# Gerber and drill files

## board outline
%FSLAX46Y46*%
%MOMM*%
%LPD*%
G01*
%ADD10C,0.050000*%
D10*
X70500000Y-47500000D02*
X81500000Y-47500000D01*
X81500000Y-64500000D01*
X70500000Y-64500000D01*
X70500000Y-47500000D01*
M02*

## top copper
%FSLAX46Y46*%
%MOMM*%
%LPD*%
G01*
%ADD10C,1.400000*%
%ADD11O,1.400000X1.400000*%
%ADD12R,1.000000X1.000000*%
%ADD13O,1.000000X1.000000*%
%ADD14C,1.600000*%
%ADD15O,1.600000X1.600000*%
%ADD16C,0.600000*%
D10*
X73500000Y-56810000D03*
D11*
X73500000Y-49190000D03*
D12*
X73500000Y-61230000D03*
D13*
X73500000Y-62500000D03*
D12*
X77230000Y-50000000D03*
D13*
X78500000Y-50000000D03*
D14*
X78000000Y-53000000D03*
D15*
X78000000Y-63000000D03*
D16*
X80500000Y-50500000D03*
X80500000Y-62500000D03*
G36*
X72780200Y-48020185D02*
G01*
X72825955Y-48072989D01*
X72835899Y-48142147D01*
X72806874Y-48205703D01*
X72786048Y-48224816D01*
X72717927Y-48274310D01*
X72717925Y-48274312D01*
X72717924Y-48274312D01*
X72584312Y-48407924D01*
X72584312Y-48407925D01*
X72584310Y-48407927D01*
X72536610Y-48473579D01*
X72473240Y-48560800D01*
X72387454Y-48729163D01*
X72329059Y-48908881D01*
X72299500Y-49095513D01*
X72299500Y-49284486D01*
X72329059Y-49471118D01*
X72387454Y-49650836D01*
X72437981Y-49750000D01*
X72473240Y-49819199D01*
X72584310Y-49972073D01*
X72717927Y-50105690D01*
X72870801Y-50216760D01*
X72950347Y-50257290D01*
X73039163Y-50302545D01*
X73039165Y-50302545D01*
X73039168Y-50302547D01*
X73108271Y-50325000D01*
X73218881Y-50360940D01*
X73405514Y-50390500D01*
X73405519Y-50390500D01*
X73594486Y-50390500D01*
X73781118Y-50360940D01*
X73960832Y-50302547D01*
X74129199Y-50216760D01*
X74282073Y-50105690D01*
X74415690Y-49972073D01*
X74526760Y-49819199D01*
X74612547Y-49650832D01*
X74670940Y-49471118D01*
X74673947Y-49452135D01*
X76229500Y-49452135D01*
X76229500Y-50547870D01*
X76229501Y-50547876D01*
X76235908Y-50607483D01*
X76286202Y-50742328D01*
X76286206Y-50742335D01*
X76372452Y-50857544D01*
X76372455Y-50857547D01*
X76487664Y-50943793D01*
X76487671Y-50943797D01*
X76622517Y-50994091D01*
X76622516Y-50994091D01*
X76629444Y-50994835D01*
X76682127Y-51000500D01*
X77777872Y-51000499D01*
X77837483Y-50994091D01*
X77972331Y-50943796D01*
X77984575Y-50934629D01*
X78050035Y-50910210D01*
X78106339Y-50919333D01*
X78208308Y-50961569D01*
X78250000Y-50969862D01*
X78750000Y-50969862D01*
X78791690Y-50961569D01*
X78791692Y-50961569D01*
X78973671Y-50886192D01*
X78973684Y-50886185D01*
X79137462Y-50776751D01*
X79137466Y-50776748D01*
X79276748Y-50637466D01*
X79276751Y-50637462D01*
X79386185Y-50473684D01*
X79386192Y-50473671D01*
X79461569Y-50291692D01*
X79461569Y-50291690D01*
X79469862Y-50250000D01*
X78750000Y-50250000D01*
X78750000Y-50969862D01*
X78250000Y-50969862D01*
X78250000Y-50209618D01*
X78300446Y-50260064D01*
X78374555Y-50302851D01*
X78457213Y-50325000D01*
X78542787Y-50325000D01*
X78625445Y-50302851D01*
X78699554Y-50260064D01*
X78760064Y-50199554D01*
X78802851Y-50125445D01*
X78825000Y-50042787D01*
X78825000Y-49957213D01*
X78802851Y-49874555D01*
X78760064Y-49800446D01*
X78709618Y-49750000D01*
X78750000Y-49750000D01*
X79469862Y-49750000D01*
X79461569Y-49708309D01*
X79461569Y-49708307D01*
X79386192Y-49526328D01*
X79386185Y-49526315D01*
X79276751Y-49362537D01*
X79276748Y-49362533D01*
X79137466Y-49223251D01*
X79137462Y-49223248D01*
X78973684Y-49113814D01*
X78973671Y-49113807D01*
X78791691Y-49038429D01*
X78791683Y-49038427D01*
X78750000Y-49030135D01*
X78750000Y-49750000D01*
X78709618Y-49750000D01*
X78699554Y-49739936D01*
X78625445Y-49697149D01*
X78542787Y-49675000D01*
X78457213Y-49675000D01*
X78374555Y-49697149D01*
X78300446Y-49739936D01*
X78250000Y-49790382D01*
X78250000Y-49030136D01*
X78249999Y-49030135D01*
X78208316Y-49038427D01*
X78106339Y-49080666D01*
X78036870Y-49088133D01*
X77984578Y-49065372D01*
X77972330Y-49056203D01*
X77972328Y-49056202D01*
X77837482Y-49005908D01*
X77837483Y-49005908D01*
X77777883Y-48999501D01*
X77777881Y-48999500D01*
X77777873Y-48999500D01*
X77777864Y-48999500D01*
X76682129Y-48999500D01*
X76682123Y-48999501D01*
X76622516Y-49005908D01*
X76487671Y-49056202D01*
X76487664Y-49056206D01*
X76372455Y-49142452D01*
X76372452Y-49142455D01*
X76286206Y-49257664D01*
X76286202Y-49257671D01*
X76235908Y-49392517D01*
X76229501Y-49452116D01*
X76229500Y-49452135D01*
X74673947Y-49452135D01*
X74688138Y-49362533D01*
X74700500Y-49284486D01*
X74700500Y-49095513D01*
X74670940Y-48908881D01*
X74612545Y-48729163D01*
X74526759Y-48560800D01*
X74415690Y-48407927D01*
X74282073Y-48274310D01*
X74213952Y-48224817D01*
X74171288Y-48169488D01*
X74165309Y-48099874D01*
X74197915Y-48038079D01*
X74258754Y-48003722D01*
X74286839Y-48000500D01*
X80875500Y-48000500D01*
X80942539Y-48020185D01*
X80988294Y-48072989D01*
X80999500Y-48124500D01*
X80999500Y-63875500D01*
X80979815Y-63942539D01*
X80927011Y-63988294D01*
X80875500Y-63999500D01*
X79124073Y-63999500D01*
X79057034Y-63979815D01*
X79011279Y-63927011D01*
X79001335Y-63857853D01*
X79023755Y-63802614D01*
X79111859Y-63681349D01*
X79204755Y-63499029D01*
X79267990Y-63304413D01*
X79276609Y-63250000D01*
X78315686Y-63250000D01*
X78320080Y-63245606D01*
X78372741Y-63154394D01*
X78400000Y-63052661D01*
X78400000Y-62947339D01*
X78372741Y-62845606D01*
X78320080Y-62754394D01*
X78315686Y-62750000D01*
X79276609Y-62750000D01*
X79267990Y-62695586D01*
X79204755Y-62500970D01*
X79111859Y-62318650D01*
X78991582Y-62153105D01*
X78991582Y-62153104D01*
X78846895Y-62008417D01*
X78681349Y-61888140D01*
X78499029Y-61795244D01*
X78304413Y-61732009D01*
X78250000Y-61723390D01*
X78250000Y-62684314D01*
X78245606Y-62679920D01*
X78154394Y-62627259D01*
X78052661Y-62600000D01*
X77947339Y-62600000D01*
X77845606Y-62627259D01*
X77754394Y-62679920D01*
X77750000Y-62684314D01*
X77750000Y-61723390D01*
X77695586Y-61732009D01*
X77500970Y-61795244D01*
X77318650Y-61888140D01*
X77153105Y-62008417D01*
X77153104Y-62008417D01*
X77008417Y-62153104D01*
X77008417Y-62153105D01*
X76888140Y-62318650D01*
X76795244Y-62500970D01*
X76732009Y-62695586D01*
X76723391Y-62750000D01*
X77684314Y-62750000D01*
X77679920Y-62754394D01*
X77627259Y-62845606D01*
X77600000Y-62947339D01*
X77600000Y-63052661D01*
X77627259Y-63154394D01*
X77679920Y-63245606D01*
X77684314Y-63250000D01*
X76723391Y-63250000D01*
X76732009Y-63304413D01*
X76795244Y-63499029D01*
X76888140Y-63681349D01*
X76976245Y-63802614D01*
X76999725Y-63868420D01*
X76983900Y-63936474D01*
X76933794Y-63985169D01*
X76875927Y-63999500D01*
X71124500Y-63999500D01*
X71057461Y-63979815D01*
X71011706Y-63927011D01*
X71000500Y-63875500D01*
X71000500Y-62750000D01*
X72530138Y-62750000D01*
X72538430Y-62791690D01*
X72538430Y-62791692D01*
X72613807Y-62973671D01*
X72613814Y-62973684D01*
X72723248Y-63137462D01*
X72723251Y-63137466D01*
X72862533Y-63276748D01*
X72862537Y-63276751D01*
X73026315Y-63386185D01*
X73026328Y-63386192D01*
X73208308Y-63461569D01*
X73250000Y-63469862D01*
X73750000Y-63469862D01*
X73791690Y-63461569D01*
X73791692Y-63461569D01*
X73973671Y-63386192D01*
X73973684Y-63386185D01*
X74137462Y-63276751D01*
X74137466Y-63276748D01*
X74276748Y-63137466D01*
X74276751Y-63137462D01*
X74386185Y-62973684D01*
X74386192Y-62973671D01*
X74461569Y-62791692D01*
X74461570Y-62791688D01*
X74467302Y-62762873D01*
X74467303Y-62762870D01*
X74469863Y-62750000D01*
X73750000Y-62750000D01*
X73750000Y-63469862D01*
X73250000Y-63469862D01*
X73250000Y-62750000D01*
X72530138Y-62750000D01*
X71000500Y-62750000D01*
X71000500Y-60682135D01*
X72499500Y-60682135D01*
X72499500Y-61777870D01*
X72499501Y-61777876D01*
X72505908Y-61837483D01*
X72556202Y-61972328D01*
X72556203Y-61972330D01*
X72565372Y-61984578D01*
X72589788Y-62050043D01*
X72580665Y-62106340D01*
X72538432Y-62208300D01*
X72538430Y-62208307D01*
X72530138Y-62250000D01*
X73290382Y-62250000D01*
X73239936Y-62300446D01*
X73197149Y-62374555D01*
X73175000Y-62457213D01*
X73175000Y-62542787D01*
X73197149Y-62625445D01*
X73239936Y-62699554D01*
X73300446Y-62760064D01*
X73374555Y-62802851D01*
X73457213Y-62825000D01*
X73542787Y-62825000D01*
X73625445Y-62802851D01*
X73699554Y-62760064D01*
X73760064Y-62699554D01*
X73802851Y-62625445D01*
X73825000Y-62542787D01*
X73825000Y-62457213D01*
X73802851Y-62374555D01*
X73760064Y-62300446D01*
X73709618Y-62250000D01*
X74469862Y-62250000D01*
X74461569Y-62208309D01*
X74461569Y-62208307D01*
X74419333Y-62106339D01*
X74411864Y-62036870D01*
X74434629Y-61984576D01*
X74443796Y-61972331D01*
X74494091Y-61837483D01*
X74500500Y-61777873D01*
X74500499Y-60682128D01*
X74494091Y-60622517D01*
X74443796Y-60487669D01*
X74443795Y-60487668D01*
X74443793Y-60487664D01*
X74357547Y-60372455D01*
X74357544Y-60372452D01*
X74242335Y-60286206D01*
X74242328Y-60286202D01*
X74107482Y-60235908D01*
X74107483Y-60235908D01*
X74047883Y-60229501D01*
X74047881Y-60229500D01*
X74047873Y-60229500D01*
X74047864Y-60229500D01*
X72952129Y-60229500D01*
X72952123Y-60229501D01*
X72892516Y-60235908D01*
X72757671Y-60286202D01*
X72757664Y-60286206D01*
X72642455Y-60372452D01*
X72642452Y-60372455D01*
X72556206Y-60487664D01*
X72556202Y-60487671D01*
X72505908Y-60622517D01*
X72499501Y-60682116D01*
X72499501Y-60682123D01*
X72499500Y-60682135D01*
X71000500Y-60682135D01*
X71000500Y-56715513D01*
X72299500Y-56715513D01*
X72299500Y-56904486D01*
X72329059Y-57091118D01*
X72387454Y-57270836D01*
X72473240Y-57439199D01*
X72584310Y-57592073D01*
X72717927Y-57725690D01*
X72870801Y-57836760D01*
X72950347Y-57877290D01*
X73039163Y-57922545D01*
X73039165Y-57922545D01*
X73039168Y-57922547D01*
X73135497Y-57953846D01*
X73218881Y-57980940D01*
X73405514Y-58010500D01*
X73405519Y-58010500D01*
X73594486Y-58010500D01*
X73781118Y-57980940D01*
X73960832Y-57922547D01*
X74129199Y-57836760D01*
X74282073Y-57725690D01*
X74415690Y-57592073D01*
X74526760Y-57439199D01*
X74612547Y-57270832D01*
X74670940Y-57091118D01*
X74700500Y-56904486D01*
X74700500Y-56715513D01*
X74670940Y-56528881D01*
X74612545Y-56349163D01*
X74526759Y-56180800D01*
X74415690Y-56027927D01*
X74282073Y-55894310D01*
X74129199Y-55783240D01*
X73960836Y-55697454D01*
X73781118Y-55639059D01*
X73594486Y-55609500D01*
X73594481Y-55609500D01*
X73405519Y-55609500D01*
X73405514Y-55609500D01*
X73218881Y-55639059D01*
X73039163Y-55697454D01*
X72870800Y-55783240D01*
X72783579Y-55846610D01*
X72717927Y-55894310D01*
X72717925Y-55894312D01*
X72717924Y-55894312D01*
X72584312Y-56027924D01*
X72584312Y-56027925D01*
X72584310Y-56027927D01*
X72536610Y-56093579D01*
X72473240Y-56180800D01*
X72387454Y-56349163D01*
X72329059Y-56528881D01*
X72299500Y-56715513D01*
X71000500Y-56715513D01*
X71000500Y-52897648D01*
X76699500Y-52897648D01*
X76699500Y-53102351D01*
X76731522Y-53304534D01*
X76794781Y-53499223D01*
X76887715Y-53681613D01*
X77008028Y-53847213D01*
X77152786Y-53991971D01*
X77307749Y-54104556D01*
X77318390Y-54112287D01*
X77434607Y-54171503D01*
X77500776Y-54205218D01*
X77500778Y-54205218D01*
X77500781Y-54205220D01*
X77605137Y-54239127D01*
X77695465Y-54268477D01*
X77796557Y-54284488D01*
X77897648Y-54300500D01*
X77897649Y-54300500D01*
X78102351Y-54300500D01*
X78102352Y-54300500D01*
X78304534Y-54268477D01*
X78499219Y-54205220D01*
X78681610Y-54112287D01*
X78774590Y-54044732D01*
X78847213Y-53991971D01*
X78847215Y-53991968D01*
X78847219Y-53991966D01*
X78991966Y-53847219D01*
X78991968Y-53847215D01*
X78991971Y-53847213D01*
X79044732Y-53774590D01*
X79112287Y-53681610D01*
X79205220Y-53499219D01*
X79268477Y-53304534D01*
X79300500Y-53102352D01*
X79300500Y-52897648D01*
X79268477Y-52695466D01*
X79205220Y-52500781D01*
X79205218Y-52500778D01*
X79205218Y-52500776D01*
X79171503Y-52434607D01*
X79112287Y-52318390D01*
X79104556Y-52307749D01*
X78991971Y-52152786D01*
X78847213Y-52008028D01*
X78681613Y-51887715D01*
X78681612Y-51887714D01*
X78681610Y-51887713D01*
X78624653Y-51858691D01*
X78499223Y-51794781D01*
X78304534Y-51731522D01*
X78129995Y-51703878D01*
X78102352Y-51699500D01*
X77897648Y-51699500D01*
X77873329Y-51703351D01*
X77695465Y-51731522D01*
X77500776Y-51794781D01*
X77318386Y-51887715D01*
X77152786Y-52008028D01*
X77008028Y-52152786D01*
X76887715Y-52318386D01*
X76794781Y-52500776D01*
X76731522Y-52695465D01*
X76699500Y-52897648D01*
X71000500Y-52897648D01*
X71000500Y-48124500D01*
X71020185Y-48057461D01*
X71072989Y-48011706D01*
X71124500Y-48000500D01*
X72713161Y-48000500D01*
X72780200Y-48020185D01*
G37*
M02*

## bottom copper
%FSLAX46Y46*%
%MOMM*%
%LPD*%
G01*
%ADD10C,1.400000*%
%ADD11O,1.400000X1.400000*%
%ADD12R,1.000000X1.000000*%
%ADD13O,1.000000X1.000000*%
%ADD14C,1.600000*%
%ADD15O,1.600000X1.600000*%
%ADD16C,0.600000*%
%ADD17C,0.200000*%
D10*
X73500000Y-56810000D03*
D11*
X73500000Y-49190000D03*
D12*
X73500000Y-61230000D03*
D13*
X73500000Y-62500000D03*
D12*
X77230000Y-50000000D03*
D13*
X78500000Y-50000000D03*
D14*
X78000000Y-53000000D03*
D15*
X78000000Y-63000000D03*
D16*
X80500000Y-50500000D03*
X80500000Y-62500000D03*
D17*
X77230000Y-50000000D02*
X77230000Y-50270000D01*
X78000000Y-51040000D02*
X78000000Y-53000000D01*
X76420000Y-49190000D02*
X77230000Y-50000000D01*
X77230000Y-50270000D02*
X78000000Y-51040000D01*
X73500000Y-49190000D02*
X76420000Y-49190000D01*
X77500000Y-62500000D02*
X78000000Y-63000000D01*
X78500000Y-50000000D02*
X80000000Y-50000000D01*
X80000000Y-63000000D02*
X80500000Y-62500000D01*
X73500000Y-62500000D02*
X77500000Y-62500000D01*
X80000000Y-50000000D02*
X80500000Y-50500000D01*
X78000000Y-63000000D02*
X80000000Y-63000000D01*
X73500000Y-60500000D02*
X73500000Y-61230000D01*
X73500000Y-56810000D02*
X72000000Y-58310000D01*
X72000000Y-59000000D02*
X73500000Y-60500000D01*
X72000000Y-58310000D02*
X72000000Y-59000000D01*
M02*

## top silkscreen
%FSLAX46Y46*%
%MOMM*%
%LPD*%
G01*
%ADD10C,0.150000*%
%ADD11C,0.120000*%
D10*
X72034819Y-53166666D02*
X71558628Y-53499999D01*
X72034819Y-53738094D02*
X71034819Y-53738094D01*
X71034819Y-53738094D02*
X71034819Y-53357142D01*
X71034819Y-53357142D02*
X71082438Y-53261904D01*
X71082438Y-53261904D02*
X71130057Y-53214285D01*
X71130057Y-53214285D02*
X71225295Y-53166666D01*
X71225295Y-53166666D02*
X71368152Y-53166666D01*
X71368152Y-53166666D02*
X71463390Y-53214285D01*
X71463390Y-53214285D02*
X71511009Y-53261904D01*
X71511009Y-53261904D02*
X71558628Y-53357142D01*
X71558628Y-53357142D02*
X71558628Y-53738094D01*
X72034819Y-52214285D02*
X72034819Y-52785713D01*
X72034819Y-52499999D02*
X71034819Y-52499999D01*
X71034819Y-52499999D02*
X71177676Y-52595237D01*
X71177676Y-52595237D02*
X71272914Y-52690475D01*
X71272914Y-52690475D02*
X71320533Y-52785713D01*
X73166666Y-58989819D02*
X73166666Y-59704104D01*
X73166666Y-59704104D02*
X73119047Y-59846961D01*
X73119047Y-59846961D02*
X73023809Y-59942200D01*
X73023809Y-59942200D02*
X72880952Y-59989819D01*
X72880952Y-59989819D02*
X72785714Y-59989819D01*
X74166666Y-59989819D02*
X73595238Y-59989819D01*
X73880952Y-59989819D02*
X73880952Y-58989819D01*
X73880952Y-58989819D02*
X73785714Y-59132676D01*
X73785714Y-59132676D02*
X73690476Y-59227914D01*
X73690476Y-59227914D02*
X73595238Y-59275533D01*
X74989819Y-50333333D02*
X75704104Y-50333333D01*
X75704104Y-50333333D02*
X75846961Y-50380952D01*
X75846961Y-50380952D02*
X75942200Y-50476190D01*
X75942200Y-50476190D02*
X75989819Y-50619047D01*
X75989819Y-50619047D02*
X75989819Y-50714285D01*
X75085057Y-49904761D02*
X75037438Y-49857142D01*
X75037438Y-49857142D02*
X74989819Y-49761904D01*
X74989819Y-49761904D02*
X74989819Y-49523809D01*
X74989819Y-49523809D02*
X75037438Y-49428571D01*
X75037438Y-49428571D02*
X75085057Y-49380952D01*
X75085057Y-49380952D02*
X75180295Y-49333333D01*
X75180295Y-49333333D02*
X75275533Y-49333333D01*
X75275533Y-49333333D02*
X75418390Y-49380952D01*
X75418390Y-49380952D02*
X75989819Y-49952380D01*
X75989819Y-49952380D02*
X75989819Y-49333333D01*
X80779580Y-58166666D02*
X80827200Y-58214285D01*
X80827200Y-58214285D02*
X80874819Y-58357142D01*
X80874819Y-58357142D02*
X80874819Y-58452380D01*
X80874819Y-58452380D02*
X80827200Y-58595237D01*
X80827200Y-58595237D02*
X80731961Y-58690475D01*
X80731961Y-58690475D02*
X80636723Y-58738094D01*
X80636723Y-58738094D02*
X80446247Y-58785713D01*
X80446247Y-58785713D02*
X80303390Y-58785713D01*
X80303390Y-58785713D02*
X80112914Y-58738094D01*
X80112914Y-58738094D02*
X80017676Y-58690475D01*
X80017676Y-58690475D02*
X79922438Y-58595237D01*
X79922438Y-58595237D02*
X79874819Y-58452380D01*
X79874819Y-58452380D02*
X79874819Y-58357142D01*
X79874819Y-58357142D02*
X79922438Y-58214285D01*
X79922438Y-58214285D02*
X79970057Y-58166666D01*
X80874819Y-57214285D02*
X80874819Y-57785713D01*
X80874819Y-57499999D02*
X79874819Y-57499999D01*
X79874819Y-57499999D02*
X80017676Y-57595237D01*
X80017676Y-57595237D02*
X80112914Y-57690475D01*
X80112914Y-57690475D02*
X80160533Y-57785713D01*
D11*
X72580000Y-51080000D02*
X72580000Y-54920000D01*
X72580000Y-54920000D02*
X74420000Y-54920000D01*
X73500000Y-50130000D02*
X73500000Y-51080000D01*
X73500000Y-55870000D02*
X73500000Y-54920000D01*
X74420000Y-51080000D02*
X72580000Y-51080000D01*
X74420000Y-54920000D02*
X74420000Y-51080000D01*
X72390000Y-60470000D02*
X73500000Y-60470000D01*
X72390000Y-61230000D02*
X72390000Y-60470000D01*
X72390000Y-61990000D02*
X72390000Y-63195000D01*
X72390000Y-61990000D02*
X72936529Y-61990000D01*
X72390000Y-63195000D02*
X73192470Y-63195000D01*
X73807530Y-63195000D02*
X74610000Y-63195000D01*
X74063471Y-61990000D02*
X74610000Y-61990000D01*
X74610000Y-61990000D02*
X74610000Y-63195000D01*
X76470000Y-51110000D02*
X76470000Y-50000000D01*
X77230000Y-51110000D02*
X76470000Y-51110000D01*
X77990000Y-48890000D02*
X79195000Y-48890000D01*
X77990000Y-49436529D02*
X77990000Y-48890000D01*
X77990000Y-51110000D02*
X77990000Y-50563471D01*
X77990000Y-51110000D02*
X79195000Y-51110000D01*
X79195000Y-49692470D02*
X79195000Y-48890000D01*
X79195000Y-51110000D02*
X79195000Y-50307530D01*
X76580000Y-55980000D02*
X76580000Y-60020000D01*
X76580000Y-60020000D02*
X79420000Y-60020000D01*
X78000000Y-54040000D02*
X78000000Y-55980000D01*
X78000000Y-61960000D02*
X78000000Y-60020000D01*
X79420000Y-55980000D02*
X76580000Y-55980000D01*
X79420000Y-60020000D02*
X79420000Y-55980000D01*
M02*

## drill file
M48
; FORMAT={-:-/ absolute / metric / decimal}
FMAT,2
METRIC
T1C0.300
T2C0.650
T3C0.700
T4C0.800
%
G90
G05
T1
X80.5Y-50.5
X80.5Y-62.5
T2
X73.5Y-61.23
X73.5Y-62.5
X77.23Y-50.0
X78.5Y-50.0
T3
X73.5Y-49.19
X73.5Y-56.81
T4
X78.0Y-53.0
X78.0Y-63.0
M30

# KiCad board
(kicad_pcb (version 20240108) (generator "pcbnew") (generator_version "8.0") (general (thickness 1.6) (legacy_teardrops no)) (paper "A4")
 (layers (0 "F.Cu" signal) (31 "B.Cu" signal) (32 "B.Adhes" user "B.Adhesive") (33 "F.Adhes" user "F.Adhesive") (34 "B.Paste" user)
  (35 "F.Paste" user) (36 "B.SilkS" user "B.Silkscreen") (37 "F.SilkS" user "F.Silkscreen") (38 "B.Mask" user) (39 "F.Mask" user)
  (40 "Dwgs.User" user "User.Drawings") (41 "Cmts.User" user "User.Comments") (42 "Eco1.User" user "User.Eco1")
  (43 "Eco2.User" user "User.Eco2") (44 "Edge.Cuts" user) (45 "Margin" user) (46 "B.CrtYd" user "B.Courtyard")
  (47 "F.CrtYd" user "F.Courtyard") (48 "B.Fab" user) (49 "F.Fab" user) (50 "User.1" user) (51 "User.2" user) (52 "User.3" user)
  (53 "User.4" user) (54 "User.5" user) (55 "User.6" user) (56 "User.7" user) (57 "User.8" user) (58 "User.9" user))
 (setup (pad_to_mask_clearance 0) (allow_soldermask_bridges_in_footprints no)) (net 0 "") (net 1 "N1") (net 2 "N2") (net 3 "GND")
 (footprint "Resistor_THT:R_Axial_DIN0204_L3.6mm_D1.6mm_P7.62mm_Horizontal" (layer "F.Cu") (at 73.5 56.81 90)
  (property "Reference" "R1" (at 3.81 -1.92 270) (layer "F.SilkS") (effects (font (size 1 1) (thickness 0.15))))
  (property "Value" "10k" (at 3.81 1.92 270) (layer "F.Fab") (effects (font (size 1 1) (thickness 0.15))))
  (fp_line (start 5.73 -0.92) (end 1.89 -0.92) (stroke (width 0.12) (type solid)) (layer "F.SilkS"))
  (fp_line (start 1.89 -0.92) (end 1.89 0.92) (stroke (width 0.12) (type solid)) (layer "F.SilkS"))
  (fp_line (start 6.68 0) (end 5.73 0) (stroke (width 0.12) (type solid)) (layer "F.SilkS"))
  (fp_line (start 0.94 0) (end 1.89 0) (stroke (width 0.12) (type solid)) (layer "F.SilkS"))
  (fp_line (start 5.73 0.92) (end 5.73 -0.92) (stroke (width 0.12) (type solid)) (layer "F.SilkS"))
  (fp_line (start 1.89 0.92) (end 5.73 0.92) (stroke (width 0.12) (type solid)) (layer "F.SilkS"))
  (pad "1" thru_hole circle (at 0 0 90) (size 1.4 1.4) (drill 0.7) (layers "*.Cu" "*.Mask") (remove_unused_layers no) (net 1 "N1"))
  (pad "2" thru_hole oval (at 7.62 0 90) (size 1.4 1.4) (drill 0.7) (layers "*.Cu" "*.Mask") (remove_unused_layers no) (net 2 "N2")))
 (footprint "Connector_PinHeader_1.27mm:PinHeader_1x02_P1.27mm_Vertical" (layer "F.Cu") (at 73.5 61.23)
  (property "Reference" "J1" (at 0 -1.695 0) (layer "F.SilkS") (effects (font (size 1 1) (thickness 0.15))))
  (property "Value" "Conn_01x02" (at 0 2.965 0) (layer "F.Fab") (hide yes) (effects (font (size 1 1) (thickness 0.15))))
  (fp_line (start -1.11 -0.76) (end 0 -0.76) (stroke (width 0.12) (type solid)) (layer "F.SilkS"))
  (fp_line (start -1.11 0) (end -1.11 -0.76) (stroke (width 0.12) (type solid)) (layer "F.SilkS"))
  (fp_line (start -1.11 0.76) (end -1.11 1.965) (stroke (width 0.12) (type solid)) (layer "F.SilkS"))
  (fp_line (start -1.11 0.76) (end -0.563471 0.76) (stroke (width 0.12) (type solid)) (layer "F.SilkS"))
  (fp_line (start -1.11 1.965) (end -0.30753 1.965) (stroke (width 0.12) (type solid)) (layer "F.SilkS"))
  (fp_line (start 0.30753 1.965) (end 1.11 1.965) (stroke (width 0.12) (type solid)) (layer "F.SilkS"))
  (fp_line (start 0.563471 0.76) (end 1.11 0.76) (stroke (width 0.12) (type solid)) (layer "F.SilkS"))
  (fp_line (start 1.11 0.76) (end 1.11 1.965) (stroke (width 0.12) (type solid)) (layer "F.SilkS"))
  (pad "1" thru_hole rect (at 0 0) (size 1 1) (drill 0.65) (layers "*.Cu" "*.Mask") (remove_unused_layers no) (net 1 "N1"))
  (pad "2" thru_hole oval (at 0 1.27) (size 1 1) (drill 0.65) (layers "*.Cu" "*.Mask") (remove_unused_layers no) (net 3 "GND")))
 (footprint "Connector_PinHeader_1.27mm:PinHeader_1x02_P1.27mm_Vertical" (layer "F.Cu") (at 77.23 50 90)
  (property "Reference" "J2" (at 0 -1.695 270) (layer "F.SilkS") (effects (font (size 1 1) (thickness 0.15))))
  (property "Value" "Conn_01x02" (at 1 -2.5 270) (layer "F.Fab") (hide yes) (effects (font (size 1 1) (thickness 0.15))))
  (fp_line (start -1.11 -0.76) (end 0 -0.76) (stroke (width 0.12) (type solid)) (layer "F.SilkS"))
  (fp_line (start -1.11 0) (end -1.11 -0.76) (stroke (width 0.12) (type solid)) (layer "F.SilkS"))
  (fp_line (start 1.11 0.76) (end 1.11 1.965) (stroke (width 0.12) (type solid)) (layer "F.SilkS"))
  (fp_line (start 0.563471 0.76) (end 1.11 0.76) (stroke (width 0.12) (type solid)) (layer "F.SilkS"))
  (fp_line (start -1.11 0.76) (end -0.563471 0.76) (stroke (width 0.12) (type solid)) (layer "F.SilkS"))
  (fp_line (start -1.11 0.76) (end -1.11 1.965) (stroke (width 0.12) (type solid)) (layer "F.SilkS"))
  (fp_line (start 0.30753 1.965) (end 1.11 1.965) (stroke (width 0.12) (type solid)) (layer "F.SilkS"))
  (fp_line (start -1.11 1.965) (end -0.30753 1.965) (stroke (width 0.12) (type solid)) (layer "F.SilkS"))
  (pad "1" thru_hole rect (at 0 0 90) (size 1 1) (drill 0.65) (layers "*.Cu" "*.Mask") (remove_unused_layers no) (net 2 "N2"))
  (pad "2" thru_hole oval (at 0 1.27 90) (size 1 1) (drill 0.65) (layers "*.Cu" "*.Mask") (remove_unused_layers no) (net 3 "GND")))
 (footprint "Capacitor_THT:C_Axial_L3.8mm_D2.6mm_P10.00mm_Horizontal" (layer "F.Cu") (at 78 53 -90)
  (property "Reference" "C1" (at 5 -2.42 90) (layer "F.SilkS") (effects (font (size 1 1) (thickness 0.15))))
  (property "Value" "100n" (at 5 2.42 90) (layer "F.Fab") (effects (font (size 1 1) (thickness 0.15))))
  (fp_line (start 2.98 1.42) (end 7.02 1.42) (stroke (width 0.12) (type solid)) (layer "F.SilkS"))
  (fp_line (start 7.02 1.42) (end 7.02 -1.42) (stroke (width 0.12) (type solid)) (layer "F.SilkS"))
  (fp_line (start 1.04 0) (end 2.98 0) (stroke (width 0.12) (type solid)) (layer "F.SilkS"))
  (fp_line (start 8.96 0) (end 7.02 0) (stroke (width 0.12) (type solid)) (layer "F.SilkS"))
  (fp_line (start 2.98 -1.42) (end 2.98 1.42) (stroke (width 0.12) (type solid)) (layer "F.SilkS"))
  (fp_line (start 7.02 -1.42) (end 2.98 -1.42) (stroke (width 0.12) (type solid)) (layer "F.SilkS"))
  (pad "1" thru_hole circle (at 0 0 270) (size 1.6 1.6) (drill 0.8) (layers "*.Cu" "*.Mask") (remove_unused_layers no) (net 2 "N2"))
  (pad "2" thru_hole oval (at 10 0 270) (size 1.6 1.6) (drill 0.8) (layers "*.Cu" "*.Mask") (remove_unused_layers no) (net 3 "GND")))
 (gr_rect (start 70.5 47.5) (end 81.5 64.5) (stroke (width 0.05) (type default)) (fill none) (layer "Edge.Cuts"))
 (segment (start 77.23 50) (end 77.23 50.27) (width 0.2) (layer "B.Cu") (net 2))
 (segment (start 78 51.04) (end 78 53) (width 0.2) (layer "B.Cu") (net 2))
 (segment (start 76.42 49.19) (end 77.23 50) (width 0.2) (layer "B.Cu") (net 2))
 (segment (start 77.23 50.27) (end 78 51.04) (width 0.2) (layer "B.Cu") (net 2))
 (segment (start 73.5 49.19) (end 76.42 49.19) (width 0.2) (layer "B.Cu") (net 2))
 (via (at 80.5 50.5) (size 0.6) (drill 0.3) (layers "F.Cu" "B.Cu") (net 3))
 (via (at 80.5 62.5) (size 0.6) (drill 0.3) (layers "F.Cu" "B.Cu") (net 3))
 (segment (start 77.5 62.5) (end 78 63) (width 0.2) (layer "B.Cu") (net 3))
 (segment (start 78.5 50) (end 80 50) (width 0.2) (layer "B.Cu") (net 3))
 (segment (start 80 63) (end 80.5 62.5) (width 0.2) (layer "B.Cu") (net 3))
 (segment (start 73.5 62.5) (end 77.5 62.5) (width 0.2) (layer "B.Cu") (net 3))
 (segment (start 80 50) (end 80.5 50.5) (width 0.2) (layer "B.Cu") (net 3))
 (segment (start 78 63) (end 80 63) (width 0.2) (layer "B.Cu") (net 3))
 (segment (start 73.5 60.5) (end 73.5 61.23) (width 0.2) (layer "B.Cu") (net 1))
 (segment (start 73.5 56.81) (end 72 58.31) (width 0.2) (layer "B.Cu") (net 1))
 (segment (start 72 59) (end 73.5 60.5) (width 0.2) (layer "B.Cu") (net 1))
 (segment (start 72 58.31) (end 72 59) (width 0.2) (layer "B.Cu") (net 1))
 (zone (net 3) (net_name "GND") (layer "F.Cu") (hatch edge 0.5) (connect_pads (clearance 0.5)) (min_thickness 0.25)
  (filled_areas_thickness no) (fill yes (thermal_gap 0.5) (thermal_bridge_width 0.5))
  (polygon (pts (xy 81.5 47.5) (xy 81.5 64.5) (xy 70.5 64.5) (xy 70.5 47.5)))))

